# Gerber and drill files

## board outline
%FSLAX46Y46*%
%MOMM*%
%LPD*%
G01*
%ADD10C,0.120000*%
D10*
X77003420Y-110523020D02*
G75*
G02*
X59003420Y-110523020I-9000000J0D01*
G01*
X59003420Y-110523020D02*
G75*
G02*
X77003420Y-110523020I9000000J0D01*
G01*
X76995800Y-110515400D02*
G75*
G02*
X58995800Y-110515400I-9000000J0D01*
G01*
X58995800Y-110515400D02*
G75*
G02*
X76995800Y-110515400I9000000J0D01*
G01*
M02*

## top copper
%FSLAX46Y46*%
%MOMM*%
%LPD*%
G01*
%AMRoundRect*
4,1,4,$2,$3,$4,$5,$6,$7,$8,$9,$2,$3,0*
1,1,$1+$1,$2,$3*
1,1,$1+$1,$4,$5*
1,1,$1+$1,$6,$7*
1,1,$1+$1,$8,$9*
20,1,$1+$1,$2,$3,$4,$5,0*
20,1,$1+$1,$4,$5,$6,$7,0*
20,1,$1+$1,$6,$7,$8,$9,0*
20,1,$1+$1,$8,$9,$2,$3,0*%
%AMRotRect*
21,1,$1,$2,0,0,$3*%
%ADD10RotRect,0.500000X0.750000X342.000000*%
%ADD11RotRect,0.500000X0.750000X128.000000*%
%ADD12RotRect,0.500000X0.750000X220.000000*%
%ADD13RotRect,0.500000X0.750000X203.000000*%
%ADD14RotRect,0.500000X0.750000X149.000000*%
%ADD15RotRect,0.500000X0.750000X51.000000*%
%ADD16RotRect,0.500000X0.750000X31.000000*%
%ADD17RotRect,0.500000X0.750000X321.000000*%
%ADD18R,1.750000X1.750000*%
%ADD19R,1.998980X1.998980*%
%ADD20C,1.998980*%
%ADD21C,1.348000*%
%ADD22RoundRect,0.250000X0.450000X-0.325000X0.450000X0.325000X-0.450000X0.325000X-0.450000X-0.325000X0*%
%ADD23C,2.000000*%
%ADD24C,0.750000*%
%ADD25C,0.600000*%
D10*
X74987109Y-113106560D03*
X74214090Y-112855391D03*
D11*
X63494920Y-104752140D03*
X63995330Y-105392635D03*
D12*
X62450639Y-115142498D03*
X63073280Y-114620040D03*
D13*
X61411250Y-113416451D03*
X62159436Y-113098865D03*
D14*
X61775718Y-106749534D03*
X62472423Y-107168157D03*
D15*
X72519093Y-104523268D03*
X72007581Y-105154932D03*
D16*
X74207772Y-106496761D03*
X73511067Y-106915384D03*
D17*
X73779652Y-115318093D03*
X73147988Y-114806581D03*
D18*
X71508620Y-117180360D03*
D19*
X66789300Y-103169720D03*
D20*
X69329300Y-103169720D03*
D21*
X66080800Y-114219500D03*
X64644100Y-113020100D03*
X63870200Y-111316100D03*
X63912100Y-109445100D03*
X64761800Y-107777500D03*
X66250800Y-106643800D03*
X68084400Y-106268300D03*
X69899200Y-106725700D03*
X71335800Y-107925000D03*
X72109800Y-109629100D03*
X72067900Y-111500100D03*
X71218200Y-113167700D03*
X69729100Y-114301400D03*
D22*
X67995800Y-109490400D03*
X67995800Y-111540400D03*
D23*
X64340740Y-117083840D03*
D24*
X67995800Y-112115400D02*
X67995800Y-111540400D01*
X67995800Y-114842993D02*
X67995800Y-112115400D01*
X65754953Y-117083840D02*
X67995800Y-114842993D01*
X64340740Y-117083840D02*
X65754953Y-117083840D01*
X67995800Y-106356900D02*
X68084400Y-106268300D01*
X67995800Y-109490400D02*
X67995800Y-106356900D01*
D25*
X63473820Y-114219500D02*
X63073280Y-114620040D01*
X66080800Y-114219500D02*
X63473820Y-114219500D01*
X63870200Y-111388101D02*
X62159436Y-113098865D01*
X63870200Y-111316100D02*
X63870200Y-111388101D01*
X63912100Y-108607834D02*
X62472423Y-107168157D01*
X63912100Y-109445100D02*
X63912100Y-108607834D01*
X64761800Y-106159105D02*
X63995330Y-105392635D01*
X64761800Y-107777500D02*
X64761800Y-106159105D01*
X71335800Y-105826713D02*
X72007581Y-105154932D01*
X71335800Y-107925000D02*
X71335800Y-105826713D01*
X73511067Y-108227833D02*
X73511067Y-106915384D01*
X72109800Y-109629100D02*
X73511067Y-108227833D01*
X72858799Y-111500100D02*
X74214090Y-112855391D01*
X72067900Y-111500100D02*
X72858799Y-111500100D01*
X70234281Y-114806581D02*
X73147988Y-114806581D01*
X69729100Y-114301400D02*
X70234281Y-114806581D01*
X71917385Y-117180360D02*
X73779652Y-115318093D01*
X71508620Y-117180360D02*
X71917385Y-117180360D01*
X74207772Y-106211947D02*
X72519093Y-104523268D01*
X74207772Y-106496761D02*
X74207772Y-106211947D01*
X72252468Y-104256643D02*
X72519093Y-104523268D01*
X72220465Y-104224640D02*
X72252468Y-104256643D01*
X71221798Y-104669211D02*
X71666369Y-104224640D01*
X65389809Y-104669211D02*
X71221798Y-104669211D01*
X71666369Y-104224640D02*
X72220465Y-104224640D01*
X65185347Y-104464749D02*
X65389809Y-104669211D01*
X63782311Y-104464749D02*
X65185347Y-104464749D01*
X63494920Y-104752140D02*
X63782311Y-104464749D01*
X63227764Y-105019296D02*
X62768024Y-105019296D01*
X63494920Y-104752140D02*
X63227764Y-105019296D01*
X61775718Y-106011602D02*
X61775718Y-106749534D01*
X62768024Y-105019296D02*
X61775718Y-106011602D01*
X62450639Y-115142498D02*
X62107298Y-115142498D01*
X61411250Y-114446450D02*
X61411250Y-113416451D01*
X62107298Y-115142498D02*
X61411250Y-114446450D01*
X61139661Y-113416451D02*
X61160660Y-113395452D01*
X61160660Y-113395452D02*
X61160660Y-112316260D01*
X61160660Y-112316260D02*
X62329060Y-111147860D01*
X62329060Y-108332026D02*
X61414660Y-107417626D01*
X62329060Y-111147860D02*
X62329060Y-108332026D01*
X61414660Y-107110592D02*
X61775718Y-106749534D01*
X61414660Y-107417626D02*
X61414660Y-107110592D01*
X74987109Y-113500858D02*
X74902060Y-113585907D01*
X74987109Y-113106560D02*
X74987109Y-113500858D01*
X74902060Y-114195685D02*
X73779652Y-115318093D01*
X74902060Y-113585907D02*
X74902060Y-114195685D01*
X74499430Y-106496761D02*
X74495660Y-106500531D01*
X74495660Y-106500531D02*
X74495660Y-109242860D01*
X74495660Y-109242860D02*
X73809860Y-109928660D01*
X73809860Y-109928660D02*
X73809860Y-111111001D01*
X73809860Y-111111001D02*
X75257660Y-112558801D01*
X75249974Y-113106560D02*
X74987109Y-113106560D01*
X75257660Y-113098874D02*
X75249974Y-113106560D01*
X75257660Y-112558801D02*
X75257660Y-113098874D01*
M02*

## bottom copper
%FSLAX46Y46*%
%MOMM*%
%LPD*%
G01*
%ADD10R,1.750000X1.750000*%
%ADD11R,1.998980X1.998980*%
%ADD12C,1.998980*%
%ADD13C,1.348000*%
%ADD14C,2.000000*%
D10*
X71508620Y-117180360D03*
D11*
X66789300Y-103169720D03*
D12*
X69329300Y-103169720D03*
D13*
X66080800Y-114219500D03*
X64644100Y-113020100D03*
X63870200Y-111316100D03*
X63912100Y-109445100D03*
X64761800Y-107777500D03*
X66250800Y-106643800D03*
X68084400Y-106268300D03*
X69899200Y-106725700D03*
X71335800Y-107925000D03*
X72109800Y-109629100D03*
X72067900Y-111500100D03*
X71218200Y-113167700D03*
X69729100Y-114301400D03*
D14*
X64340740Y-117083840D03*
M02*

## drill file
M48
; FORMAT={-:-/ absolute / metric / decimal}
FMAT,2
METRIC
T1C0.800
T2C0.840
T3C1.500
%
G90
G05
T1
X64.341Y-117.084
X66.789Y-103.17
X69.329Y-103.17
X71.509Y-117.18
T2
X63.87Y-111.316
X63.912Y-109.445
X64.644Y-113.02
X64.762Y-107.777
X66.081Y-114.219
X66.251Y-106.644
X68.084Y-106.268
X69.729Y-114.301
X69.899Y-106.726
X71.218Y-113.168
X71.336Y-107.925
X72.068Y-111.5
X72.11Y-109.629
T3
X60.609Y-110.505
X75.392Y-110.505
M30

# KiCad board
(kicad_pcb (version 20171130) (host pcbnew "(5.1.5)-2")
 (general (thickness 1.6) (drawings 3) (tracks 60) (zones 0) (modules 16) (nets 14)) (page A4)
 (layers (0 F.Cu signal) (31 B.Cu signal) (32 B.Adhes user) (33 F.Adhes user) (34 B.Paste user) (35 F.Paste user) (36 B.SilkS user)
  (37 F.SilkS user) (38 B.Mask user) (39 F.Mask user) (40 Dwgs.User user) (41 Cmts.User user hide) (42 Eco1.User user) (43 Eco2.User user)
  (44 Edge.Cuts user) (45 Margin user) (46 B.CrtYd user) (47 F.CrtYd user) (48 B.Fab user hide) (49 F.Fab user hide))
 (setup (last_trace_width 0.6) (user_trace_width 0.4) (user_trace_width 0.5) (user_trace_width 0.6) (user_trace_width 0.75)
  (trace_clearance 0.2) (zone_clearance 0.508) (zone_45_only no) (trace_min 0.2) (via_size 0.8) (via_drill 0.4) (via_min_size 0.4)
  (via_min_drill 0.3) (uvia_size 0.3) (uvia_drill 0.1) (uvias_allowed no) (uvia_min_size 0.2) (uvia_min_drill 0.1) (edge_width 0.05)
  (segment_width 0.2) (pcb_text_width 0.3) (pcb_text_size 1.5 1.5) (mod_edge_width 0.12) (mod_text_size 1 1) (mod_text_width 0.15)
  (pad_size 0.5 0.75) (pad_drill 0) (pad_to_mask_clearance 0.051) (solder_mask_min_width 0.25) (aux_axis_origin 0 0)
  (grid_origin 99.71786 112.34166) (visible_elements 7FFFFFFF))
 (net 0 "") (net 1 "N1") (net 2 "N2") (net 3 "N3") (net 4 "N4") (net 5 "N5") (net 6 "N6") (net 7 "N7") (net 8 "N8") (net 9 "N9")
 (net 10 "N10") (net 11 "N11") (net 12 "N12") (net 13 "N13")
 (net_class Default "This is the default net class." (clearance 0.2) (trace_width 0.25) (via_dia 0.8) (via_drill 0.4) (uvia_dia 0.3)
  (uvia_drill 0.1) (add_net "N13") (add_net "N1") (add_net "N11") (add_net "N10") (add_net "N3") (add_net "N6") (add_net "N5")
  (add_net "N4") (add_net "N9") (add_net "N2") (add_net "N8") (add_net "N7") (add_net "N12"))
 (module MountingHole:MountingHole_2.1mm (layer F.Cu) (at 60.60948 110.50524)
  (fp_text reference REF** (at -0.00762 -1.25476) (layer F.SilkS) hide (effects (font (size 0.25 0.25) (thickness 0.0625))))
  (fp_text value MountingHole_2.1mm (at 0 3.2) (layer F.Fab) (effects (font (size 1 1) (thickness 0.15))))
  (pad "" np_thru_hole circle (at 0 0) (size 1.5 1.5) (drill 1.5) (layers *.Cu *.Mask)))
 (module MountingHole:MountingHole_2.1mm (layer F.Cu) (at 75.39228 110.50524)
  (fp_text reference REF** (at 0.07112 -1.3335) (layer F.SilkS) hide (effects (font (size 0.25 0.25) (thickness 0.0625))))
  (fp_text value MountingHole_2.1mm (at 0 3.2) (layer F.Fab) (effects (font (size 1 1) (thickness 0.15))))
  (pad "" np_thru_hole circle (at 0 0) (size 1.5 1.5) (drill 1.5) (layers *.Cu *.Mask)))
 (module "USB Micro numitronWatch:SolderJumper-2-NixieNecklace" (layer F.Cu) (at 74.82586 113.02746 342)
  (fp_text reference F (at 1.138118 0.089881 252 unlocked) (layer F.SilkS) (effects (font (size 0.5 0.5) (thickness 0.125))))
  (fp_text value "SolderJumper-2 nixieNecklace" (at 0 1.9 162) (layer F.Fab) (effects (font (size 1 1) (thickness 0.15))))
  (pad 2 smd rect (at 0.1778 0.0254 342) (size 0.5 0.75) (layers F.Cu F.Mask) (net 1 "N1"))
  (pad 1 smd rect (at -0.635 0.0254 342) (size 0.5 0.75) (layers F.Cu F.Mask) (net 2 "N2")))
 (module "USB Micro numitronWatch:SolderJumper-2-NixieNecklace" (layer F.Cu) (at 63.584369 104.907886 128)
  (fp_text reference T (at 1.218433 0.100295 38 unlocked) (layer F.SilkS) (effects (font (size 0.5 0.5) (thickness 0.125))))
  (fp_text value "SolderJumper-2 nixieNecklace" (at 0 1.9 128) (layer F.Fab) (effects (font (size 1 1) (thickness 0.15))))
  (pad 2 smd rect (at 0.1778 0.0254 128) (size 0.5 0.75) (layers F.Cu F.Mask) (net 1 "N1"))
  (pad 1 smd rect (at -0.635 0.0254 128) (size 0.5 0.75) (layers F.Cu F.Mask) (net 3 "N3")))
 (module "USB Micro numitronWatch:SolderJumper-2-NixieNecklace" (layer F.Cu) (at 62.603169 115.047668 220)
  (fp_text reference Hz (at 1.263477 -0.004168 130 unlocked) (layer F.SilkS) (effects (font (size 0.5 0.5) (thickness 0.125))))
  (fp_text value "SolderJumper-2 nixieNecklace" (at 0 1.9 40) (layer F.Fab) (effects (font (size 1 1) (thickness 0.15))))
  (pad 2 smd rect (at 0.1778 0.0254 220) (size 0.5 0.75) (layers F.Cu F.Mask) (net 1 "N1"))
  (pad 1 smd rect (at -0.635 0.0254 220) (size 0.5 0.75) (layers F.Cu F.Mask) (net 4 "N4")))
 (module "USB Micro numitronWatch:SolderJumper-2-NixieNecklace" (layer F.Cu) (at 61.58484 113.37036 203)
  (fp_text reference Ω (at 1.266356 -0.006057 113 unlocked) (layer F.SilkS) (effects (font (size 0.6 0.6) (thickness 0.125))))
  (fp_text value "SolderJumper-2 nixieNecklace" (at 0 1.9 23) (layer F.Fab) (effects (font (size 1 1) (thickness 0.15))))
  (pad 2 smd rect (at 0.1778 0.0254 203) (size 0.5 0.75) (layers F.Cu F.Mask) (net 1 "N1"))
  (pad 1 smd rect (at -0.635 0.0254 203) (size 0.5 0.75) (layers F.Cu F.Mask) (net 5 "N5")))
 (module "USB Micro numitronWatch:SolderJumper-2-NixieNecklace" (layer F.Cu) (at 61.91504 106.86288 149)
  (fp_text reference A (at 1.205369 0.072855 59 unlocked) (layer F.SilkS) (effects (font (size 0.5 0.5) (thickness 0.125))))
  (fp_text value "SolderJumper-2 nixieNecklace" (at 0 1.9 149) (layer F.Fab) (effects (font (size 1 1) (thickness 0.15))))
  (pad 2 smd rect (at 0.1778 0.0254 149) (size 0.5 0.75) (layers F.Cu F.Mask) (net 1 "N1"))
  (pad 1 smd rect (at -0.635 0.0254 149) (size 0.5 0.75) (layers F.Cu F.Mask) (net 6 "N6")))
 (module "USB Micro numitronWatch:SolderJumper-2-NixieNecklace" (layer F.Cu) (at 72.38746 104.64546 51)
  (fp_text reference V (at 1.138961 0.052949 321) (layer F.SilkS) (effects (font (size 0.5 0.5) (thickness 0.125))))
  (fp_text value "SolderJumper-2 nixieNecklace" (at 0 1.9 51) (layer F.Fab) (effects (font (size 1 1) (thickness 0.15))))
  (pad 2 smd rect (at 0.1778 0.0254 51) (size 0.5 0.75) (layers F.Cu F.Mask) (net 1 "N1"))
  (pad 1 smd rect (at -0.635 0.0254 51) (size 0.5 0.75) (layers F.Cu F.Mask) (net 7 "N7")))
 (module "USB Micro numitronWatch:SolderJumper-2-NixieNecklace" (layer F.Cu) (at 74.042286 106.566563 31)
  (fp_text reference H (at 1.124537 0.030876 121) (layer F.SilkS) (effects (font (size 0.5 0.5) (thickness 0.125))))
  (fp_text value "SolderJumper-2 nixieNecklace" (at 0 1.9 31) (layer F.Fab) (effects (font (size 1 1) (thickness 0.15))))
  (pad 2 smd rect (at 0.1778 0.0254 31) (size 0.5 0.75) (layers F.Cu F.Mask) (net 1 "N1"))
  (pad 1 smd rect (at -0.635 0.0254 31) (size 0.5 0.75) (layers F.Cu F.Mask) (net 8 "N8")))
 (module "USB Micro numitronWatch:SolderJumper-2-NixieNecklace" (layer F.Cu) (at 73.65746 115.18646 321)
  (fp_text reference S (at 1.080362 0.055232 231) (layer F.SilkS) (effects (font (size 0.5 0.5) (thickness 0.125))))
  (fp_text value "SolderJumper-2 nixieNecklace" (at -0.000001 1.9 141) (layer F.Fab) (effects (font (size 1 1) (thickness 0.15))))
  (pad 2 smd rect (at 0.1778 0.0254 321) (size 0.5 0.75) (layers F.Cu F.Mask) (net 1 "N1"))
  (pad 1 smd rect (at -0.635 0.0254 321) (size 0.5 0.75) (layers F.Cu F.Mask) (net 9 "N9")))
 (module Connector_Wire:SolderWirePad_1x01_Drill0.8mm (layer F.Cu) (at 71.50862 117.18036)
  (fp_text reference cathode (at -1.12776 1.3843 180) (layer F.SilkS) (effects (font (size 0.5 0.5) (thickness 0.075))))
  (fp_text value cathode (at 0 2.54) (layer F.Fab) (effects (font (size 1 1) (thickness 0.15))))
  (pad 1 thru_hole rect (at 0 0) (size 1.75 1.75) (drill 0.8001) (layers *.Cu *.Mask) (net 1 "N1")))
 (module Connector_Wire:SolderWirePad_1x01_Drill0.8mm (layer F.Cu) (at 66.7893 103.16972)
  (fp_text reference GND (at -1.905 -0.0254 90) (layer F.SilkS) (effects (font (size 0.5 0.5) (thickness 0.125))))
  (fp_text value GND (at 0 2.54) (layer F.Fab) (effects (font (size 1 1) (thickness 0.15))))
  (pad 1 thru_hole rect (at 0 0) (size 1.99898 1.99898) (drill 0.8001) (layers *.Cu *.Mask) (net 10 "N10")))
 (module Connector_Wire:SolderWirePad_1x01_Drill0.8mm (layer F.Cu) (at 69.3293 103.16972)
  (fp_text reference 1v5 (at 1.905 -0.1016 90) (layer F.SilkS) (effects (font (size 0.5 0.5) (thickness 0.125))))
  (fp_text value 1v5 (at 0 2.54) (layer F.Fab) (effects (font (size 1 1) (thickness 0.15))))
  (pad 1 thru_hole circle (at 0 0) (size 1.99898 1.99898) (drill 0.8001) (layers *.Cu *.Mask) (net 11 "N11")))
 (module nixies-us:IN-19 (layer F.Cu) (at 67.9958 110.5154)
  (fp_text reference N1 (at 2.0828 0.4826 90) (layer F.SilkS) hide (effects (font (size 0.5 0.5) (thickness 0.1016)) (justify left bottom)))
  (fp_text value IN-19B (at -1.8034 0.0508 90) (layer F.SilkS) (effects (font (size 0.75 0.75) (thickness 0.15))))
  (pad 14 thru_hole circle (at -1.915 3.7041 333) (size 1.348 1.348) (drill 0.84) (layers *.Cu *.Mask) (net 4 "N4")
   (solder_mask_margin 0.1016))
  (pad 13 thru_hole circle (at -3.3517 2.5047 333) (size 1.348 1.348) (drill 0.84) (layers *.Cu *.Mask) (solder_mask_margin 0.1016))
  (pad 12 thru_hole circle (at -4.1256 0.8007 333) (size 1.348 1.348) (drill 0.84) (layers *.Cu *.Mask) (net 5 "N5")
   (solder_mask_margin 0.1016))
  (pad 11 thru_hole circle (at -4.0837 -1.0703 333) (size 1.348 1.348) (drill 0.84) (layers *.Cu *.Mask) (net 6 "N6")
   (solder_mask_margin 0.1016))
  (pad 10 thru_hole circle (at -3.234 -2.7379 333) (size 1.348 1.348) (drill 0.84) (layers *.Cu *.Mask) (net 3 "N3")
   (solder_mask_margin 0.1016))
  (pad 9 thru_hole circle (at -1.745 -3.8716 333) (size 1.348 1.348) (drill 0.84) (layers *.Cu *.Mask) (solder_mask_margin 0.1016))
  (pad 8 thru_hole circle (at 0.0886 -4.2471 333) (size 1.348 1.348) (drill 0.84) (layers *.Cu *.Mask) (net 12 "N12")
   (solder_mask_margin 0.1016))
  (pad 7 thru_hole circle (at 1.9034 -3.7897 333) (size 1.348 1.348) (drill 0.84) (layers *.Cu *.Mask) (solder_mask_margin 0.1016))
  (pad 6 thru_hole circle (at 3.34 -2.5904 333) (size 1.348 1.348) (drill 0.84) (layers *.Cu *.Mask) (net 7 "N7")
   (solder_mask_margin 0.1016))
  (pad 5 thru_hole circle (at 4.114 -0.8863 333) (size 1.348 1.348) (drill 0.84) (layers *.Cu *.Mask) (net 8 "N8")
   (solder_mask_margin 0.1016))
  (pad 4 thru_hole circle (at 4.0721 0.9847 333) (size 1.348 1.348) (drill 0.84) (layers *.Cu *.Mask) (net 2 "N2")
   (solder_mask_margin 0.1016))
  (pad 3 thru_hole circle (at 3.2224 2.6523 333) (size 1.348 1.348) (drill 0.84) (layers *.Cu *.Mask) (solder_mask_margin 0.1016))
  (pad 2 thru_hole circle (at 1.7333 3.786 333) (size 1.348 1.348) (drill 0.84) (layers *.Cu *.Mask) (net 9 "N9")
   (solder_mask_margin 0.1016)))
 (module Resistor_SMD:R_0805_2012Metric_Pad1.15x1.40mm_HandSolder (layer F.Cu) (at 67.9958 110.5154 90)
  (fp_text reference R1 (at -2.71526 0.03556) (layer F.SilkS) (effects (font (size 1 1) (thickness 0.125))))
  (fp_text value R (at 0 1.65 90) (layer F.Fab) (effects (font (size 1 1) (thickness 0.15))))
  (pad 2 smd roundrect (at 1.025 0 90) (size 1.15 1.4) (layers F.Cu F.Paste F.Mask) (roundrect_rratio 0.217391) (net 12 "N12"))
  (pad 1 smd roundrect (at -1.025 0 90) (size 1.15 1.4) (layers F.Cu F.Paste F.Mask) (roundrect_rratio 0.217391) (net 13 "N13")))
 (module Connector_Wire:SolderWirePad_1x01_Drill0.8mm (layer F.Cu) (at 64.34074 117.08384)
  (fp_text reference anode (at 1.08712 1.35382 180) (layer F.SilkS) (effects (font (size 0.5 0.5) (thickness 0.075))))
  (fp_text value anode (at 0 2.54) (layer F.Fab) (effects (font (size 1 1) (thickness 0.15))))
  (pad 1 thru_hole circle (at 0 0) (size 2 2) (drill 0.8001) (layers *.Cu *.Mask) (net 13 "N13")))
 (gr_circle (center 68.00342 110.52302) (end 77.00342 110.52302) (layer Edge.Cuts) (width 0.12))
 (gr_circle (center 67.9958 110.5154) (end 76.9958 110.5154) (layer Edge.Cuts) (width 0.12))
 (segment (start 67.9958 112.1154) (end 67.9958 111.5404) (width 0.75) (layer F.Cu) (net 13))
 (segment (start 67.9958 114.842993) (end 67.9958 112.1154) (width 0.75) (layer F.Cu) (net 13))
 (segment (start 65.754953 117.08384) (end 67.9958 114.842993) (width 0.75) (layer F.Cu) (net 13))
 (segment (start 64.34074 117.08384) (end 65.754953 117.08384) (width 0.75) (layer F.Cu) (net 13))
 (segment (start 67.9958 106.3569) (end 68.0844 106.2683) (width 0.75) (layer F.Cu) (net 12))
 (segment (start 67.9958 109.4904) (end 67.9958 106.3569) (width 0.75) (layer F.Cu) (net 12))
 (segment (start 63.47382 114.2195) (end 63.07328 114.62004) (width 0.6) (layer F.Cu) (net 4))
 (segment (start 66.0808 114.2195) (end 63.47382 114.2195) (width 0.6) (layer F.Cu) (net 4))
 (segment (start 63.8702 111.388101) (end 62.159436 113.098865) (width 0.6) (layer F.Cu) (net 5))
 (segment (start 63.8702 111.3161) (end 63.8702 111.388101) (width 0.6) (layer F.Cu) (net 5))
 (segment (start 63.9121 108.607834) (end 62.472423 107.168157) (width 0.6) (layer F.Cu) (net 6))
 (segment (start 63.9121 109.4451) (end 63.9121 108.607834) (width 0.6) (layer F.Cu) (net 6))
 (segment (start 64.7618 106.159105) (end 63.99533 105.392635) (width 0.6) (layer F.Cu) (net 3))
 (segment (start 64.7618 107.7775) (end 64.7618 106.159105) (width 0.6) (layer F.Cu) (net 3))
 (segment (start 71.3358 105.826713) (end 72.007581 105.154932) (width 0.6) (layer F.Cu) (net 7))
 (segment (start 71.3358 107.925) (end 71.3358 105.826713) (width 0.6) (layer F.Cu) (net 7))
 (segment (start 73.511067 108.227833) (end 73.511067 106.915384) (width 0.6) (layer F.Cu) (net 8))
 (segment (start 72.1098 109.6291) (end 73.511067 108.227833) (width 0.6) (layer F.Cu) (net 8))
 (segment (start 72.858799 111.5001) (end 74.21409 112.855391) (width 0.6) (layer F.Cu) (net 2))
 (segment (start 72.0679 111.5001) (end 72.858799 111.5001) (width 0.6) (layer F.Cu) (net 2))
 (segment (start 70.234281 114.806581) (end 73.147988 114.806581) (width 0.6) (layer F.Cu) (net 9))
 (segment (start 69.7291 114.3014) (end 70.234281 114.806581) (width 0.6) (layer F.Cu) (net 9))
 (segment (start 71.917385 117.18036) (end 73.779652 115.318093) (width 0.6) (layer F.Cu) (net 1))
 (segment (start 71.50862 117.18036) (end 71.917385 117.18036) (width 0.6) (layer F.Cu) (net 1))
 (segment (start 74.207772 106.211947) (end 72.519093 104.523268) (width 0.6) (layer F.Cu) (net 1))
 (segment (start 74.207772 106.496761) (end 74.207772 106.211947) (width 0.6) (layer F.Cu) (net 1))
 (segment (start 72.252468 104.256643) (end 72.519093 104.523268) (width 0.6) (layer F.Cu) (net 1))
 (segment (start 72.220465 104.22464) (end 72.252468 104.256643) (width 0.6) (layer F.Cu) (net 1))
 (segment (start 71.221798 104.669211) (end 71.666369 104.22464) (width 0.6) (layer F.Cu) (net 1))
 (segment (start 65.389809 104.669211) (end 71.221798 104.669211) (width 0.6) (layer F.Cu) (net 1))
 (segment (start 71.666369 104.22464) (end 72.220465 104.22464) (width 0.6) (layer F.Cu) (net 1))
 (segment (start 65.185347 104.464749) (end 65.389809 104.669211) (width 0.6) (layer F.Cu) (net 1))
 (segment (start 63.782311 104.464749) (end 65.185347 104.464749) (width 0.6) (layer F.Cu) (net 1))
 (segment (start 63.49492 104.75214) (end 63.782311 104.464749) (width 0.6) (layer F.Cu) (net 1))
 (segment (start 63.227764 105.019296) (end 62.768024 105.019296) (width 0.6) (layer F.Cu) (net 1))
 (segment (start 63.49492 104.75214) (end 63.227764 105.019296) (width 0.6) (layer F.Cu) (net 1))
 (segment (start 61.775718 106.011602) (end 61.775718 106.749534) (width 0.6) (layer F.Cu) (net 1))
 (segment (start 62.768024 105.019296) (end 61.775718 106.011602) (width 0.6) (layer F.Cu) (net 1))
 (segment (start 62.450639 115.142498) (end 62.107298 115.142498) (width 0.6) (layer F.Cu) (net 1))
 (segment (start 61.41125 114.44645) (end 61.41125 113.416451) (width 0.6) (layer F.Cu) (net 1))
 (segment (start 62.107298 115.142498) (end 61.41125 114.44645) (width 0.6) (layer F.Cu) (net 1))
 (segment (start 61.139661 113.416451) (end 61.16066 113.395452) (width 0.6) (layer F.Cu) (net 1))
 (segment (start 61.16066 113.395452) (end 61.16066 112.31626) (width 0.6) (layer F.Cu) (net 1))
 (segment (start 61.16066 112.31626) (end 62.32906 111.14786) (width 0.6) (layer F.Cu) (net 1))
 (segment (start 62.32906 108.332026) (end 61.41466 107.417626) (width 0.6) (layer F.Cu) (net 1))
 (segment (start 62.32906 111.14786) (end 62.32906 108.332026) (width 0.6) (layer F.Cu) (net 1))
 (segment (start 61.41466 107.110592) (end 61.775718 106.749534) (width 0.6) (layer F.Cu) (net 1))
 (segment (start 61.41466 107.417626) (end 61.41466 107.110592) (width 0.6) (layer F.Cu) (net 1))
 (segment (start 74.987109 113.500858) (end 74.90206 113.585907) (width 0.6) (layer F.Cu) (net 1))
 (segment (start 74.987109 113.10656) (end 74.987109 113.500858) (width 0.6) (layer F.Cu) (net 1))
 (segment (start 74.90206 114.195685) (end 73.779652 115.318093) (width 0.6) (layer F.Cu) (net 1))
 (segment (start 74.90206 113.585907) (end 74.90206 114.195685) (width 0.6) (layer F.Cu) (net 1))
 (segment (start 74.49943 106.496761) (end 74.49566 106.500531) (width 0.6) (layer F.Cu) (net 1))
 (segment (start 74.49566 106.500531) (end 74.49566 109.24286) (width 0.6) (layer F.Cu) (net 1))
 (segment (start 74.49566 109.24286) (end 73.80986 109.92866) (width 0.6) (layer F.Cu) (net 1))
 (segment (start 73.80986 109.92866) (end 73.80986 111.111001) (width 0.6) (layer F.Cu) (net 1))
 (segment (start 73.80986 111.111001) (end 75.25766 112.558801) (width 0.6) (layer F.Cu) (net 1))
 (segment (start 75.249974 113.10656) (end 74.987109 113.10656) (width 0.6) (layer F.Cu) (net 1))
 (segment (start 75.25766 113.098874) (end 75.249974 113.10656) (width 0.6) (layer F.Cu) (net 1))
 (segment (start 75.25766 112.558801) (end 75.25766 113.098874) (width 0.6) (layer F.Cu) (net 1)))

